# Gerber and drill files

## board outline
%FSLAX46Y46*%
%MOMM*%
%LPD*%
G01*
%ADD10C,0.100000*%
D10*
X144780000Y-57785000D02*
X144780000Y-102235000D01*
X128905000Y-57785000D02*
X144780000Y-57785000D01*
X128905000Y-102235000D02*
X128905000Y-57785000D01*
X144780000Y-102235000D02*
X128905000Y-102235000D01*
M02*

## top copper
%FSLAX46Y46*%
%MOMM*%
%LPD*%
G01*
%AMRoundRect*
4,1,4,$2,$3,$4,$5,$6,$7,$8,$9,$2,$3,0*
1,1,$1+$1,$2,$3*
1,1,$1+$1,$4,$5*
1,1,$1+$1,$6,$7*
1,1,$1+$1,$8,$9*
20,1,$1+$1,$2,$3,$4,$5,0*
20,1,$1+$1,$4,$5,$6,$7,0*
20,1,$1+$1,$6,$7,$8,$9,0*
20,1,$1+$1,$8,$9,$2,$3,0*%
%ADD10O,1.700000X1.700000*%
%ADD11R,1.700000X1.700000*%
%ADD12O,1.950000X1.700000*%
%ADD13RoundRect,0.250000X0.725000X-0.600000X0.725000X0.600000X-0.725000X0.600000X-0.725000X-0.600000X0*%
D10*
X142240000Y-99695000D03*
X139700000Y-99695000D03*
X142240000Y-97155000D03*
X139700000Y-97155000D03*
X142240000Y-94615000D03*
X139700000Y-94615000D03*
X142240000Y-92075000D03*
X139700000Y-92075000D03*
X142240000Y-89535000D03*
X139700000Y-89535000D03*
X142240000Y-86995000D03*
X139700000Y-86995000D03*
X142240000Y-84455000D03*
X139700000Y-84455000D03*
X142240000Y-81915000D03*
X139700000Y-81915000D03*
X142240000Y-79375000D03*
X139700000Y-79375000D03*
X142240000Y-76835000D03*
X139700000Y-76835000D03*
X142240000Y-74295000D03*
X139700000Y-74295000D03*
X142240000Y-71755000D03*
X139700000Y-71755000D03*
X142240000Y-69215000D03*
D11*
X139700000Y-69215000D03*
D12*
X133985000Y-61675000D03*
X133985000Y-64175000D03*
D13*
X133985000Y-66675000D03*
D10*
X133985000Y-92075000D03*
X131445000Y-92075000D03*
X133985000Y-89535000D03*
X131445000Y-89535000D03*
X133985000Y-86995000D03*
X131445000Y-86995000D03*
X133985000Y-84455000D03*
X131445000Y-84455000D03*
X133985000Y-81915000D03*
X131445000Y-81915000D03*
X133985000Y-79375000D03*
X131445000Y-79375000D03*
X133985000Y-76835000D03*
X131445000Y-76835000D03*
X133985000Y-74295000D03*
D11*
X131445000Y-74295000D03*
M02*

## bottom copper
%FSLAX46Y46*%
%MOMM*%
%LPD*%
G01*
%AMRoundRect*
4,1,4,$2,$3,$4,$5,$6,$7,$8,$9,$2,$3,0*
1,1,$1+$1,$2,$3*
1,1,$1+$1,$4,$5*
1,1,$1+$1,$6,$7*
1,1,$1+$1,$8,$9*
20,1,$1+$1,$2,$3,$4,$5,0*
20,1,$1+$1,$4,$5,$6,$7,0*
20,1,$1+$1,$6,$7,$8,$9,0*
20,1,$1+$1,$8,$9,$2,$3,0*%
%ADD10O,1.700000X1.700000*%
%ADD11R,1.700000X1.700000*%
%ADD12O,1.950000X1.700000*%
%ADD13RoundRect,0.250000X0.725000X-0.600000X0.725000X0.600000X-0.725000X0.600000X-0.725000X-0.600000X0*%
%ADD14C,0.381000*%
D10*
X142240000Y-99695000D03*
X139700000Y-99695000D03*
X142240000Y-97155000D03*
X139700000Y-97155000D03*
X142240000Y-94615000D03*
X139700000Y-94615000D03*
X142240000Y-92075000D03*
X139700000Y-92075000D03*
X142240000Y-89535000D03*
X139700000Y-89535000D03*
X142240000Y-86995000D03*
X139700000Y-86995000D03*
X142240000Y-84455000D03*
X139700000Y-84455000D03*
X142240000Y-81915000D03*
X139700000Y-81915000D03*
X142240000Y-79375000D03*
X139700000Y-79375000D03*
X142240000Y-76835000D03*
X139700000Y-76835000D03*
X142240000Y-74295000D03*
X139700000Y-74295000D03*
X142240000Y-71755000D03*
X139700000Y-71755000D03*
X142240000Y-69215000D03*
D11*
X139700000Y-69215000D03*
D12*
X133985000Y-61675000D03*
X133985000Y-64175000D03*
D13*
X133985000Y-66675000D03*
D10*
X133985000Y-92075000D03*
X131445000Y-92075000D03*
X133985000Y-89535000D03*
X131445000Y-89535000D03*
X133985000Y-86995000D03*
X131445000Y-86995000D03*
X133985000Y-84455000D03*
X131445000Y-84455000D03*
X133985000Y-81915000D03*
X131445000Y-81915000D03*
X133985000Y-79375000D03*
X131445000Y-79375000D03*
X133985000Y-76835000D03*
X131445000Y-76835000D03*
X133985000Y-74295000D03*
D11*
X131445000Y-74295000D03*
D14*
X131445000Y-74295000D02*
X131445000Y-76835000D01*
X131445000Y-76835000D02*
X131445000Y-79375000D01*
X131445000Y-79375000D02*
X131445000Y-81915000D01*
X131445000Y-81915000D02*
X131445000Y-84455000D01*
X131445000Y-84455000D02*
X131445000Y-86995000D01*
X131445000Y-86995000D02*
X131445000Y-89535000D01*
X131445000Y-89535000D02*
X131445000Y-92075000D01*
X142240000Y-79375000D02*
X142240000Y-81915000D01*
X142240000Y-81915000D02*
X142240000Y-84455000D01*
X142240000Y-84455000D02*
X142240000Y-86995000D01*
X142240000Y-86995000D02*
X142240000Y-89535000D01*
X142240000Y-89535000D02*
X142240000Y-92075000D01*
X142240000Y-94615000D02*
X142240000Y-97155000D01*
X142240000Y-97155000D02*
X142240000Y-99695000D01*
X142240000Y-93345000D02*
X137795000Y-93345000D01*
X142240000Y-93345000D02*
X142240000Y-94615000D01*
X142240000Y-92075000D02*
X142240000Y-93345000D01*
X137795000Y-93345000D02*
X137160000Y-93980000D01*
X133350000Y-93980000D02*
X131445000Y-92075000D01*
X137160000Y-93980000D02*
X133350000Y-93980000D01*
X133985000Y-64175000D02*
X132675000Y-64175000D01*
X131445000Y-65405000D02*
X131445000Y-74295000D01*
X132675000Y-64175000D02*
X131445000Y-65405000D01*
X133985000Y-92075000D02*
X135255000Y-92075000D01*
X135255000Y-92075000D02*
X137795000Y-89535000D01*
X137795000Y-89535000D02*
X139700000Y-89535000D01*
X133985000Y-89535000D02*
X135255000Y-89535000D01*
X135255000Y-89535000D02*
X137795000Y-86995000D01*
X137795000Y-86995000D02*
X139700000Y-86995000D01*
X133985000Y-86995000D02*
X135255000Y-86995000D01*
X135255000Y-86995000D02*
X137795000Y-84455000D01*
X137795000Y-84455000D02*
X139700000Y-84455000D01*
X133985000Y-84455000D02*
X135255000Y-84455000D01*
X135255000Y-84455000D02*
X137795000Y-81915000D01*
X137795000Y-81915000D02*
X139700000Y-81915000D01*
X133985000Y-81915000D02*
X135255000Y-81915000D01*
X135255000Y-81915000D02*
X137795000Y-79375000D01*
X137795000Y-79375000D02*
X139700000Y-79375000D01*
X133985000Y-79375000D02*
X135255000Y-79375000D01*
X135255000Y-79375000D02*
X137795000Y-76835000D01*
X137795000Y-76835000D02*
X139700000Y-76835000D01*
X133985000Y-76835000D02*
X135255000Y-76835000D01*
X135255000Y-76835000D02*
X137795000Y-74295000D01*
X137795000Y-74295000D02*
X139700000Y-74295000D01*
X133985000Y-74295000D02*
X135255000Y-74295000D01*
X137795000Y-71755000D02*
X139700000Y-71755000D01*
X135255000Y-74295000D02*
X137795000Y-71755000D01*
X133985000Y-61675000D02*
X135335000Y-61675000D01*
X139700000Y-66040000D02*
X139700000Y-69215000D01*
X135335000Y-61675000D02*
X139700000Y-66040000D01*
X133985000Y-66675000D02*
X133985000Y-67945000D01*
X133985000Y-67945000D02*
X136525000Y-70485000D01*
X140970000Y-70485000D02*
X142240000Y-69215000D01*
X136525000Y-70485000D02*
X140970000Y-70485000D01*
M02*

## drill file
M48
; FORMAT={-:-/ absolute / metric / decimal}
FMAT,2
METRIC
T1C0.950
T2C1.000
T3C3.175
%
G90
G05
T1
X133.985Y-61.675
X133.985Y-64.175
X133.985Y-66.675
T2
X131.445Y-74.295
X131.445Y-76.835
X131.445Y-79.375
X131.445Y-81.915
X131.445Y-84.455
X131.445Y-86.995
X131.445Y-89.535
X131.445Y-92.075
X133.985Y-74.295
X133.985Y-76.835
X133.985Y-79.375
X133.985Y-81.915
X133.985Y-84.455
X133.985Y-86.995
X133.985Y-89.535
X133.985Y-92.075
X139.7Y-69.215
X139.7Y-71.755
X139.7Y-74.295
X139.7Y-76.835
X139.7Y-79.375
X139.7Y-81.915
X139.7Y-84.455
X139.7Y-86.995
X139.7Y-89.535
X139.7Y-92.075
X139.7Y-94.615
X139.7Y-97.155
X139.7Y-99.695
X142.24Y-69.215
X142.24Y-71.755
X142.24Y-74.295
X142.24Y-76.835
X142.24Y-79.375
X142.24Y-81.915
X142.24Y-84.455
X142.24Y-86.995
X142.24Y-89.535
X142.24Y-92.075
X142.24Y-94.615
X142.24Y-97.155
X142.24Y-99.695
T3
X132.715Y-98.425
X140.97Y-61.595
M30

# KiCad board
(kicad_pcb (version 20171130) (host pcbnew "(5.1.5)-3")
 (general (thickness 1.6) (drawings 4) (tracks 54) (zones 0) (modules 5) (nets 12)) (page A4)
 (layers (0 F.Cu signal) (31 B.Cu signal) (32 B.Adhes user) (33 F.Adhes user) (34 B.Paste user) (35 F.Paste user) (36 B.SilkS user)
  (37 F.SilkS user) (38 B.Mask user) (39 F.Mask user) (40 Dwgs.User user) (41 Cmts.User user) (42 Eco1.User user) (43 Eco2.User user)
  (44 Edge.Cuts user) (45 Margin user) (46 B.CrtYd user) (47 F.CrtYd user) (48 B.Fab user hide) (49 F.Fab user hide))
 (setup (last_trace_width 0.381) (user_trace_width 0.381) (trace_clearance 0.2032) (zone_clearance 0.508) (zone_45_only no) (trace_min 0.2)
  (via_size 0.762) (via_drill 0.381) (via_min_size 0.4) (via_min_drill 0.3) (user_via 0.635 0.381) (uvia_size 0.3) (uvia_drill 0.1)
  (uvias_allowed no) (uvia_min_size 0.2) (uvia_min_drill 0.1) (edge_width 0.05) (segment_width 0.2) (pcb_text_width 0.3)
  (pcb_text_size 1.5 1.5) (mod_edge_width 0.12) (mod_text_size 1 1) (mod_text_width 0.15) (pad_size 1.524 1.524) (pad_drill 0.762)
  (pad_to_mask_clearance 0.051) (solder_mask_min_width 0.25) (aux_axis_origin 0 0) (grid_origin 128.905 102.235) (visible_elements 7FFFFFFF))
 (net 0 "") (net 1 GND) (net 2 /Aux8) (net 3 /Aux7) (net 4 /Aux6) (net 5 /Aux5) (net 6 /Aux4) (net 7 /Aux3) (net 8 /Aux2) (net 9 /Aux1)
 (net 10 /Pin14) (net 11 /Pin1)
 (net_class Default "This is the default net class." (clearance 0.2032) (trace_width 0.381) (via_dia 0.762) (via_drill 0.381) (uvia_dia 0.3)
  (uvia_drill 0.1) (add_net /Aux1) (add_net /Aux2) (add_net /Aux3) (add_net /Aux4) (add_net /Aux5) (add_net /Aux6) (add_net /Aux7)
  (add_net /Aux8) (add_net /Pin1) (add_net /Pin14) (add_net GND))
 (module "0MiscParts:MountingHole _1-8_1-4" (layer F.Cu) (at 132.715 98.425)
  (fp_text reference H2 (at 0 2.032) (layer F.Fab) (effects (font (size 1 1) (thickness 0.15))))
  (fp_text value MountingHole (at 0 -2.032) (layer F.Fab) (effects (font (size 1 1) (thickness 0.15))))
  (pad "" np_thru_hole circle (at 0 0) (size 3.175 3.175) (drill 3.175) (layers *.Cu *.Mask)))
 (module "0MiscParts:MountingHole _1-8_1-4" (layer F.Cu) (at 140.97 61.595)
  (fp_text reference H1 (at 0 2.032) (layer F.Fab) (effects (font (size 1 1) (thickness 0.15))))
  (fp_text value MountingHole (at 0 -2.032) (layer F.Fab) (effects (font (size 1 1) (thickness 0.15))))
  (pad "" np_thru_hole circle (at 0 0) (size 3.175 3.175) (drill 3.175) (layers *.Cu *.Mask)))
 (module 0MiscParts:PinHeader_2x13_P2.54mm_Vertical (layer F.Cu) (at 139.7 69.215)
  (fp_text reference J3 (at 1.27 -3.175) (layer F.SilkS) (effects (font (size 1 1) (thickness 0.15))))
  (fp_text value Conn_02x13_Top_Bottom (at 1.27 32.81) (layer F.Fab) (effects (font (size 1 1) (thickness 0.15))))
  (pad 26 thru_hole oval (at 2.54 30.48) (size 1.7 1.7) (drill 1) (layers *.Cu *.Mask) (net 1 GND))
  (pad 13 thru_hole oval (at 0 30.48) (size 1.7 1.7) (drill 1) (layers *.Cu *.Mask))
  (pad 25 thru_hole oval (at 2.54 27.94) (size 1.7 1.7) (drill 1) (layers *.Cu *.Mask) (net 1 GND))
  (pad 12 thru_hole oval (at 0 27.94) (size 1.7 1.7) (drill 1) (layers *.Cu *.Mask))
  (pad 24 thru_hole oval (at 2.54 25.4) (size 1.7 1.7) (drill 1) (layers *.Cu *.Mask) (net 1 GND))
  (pad 11 thru_hole oval (at 0 25.4) (size 1.7 1.7) (drill 1) (layers *.Cu *.Mask))
  (pad 23 thru_hole oval (at 2.54 22.86) (size 1.7 1.7) (drill 1) (layers *.Cu *.Mask) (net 1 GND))
  (pad 10 thru_hole oval (at 0 22.86) (size 1.7 1.7) (drill 1) (layers *.Cu *.Mask))
  (pad 22 thru_hole oval (at 2.54 20.32) (size 1.7 1.7) (drill 1) (layers *.Cu *.Mask) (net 1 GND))
  (pad 9 thru_hole oval (at 0 20.32) (size 1.7 1.7) (drill 1) (layers *.Cu *.Mask) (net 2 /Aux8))
  (pad 21 thru_hole oval (at 2.54 17.78) (size 1.7 1.7) (drill 1) (layers *.Cu *.Mask) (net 1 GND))
  (pad 8 thru_hole oval (at 0 17.78) (size 1.7 1.7) (drill 1) (layers *.Cu *.Mask) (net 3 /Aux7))
  (pad 20 thru_hole oval (at 2.54 15.24) (size 1.7 1.7) (drill 1) (layers *.Cu *.Mask) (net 1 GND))
  (pad 7 thru_hole oval (at 0 15.24) (size 1.7 1.7) (drill 1) (layers *.Cu *.Mask) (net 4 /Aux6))
  (pad 19 thru_hole oval (at 2.54 12.7) (size 1.7 1.7) (drill 1) (layers *.Cu *.Mask) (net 1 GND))
  (pad 6 thru_hole oval (at 0 12.7) (size 1.7 1.7) (drill 1) (layers *.Cu *.Mask) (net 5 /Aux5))
  (pad 18 thru_hole oval (at 2.54 10.16) (size 1.7 1.7) (drill 1) (layers *.Cu *.Mask) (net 1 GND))
  (pad 5 thru_hole oval (at 0 10.16) (size 1.7 1.7) (drill 1) (layers *.Cu *.Mask) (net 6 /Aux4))
  (pad 17 thru_hole oval (at 2.54 7.62) (size 1.7 1.7) (drill 1) (layers *.Cu *.Mask))
  (pad 4 thru_hole oval (at 0 7.62) (size 1.7 1.7) (drill 1) (layers *.Cu *.Mask) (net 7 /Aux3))
  (pad 16 thru_hole oval (at 2.54 5.08) (size 1.7 1.7) (drill 1) (layers *.Cu *.Mask))
  (pad 3 thru_hole oval (at 0 5.08) (size 1.7 1.7) (drill 1) (layers *.Cu *.Mask) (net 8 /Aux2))
  (pad 15 thru_hole oval (at 2.54 2.54) (size 1.7 1.7) (drill 1) (layers *.Cu *.Mask))
  (pad 2 thru_hole oval (at 0 2.54) (size 1.7 1.7) (drill 1) (layers *.Cu *.Mask) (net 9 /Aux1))
  (pad 14 thru_hole oval (at 2.54 0) (size 1.7 1.7) (drill 1) (layers *.Cu *.Mask) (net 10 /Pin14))
  (pad 1 thru_hole rect (at 0 0) (size 1.7 1.7) (drill 1) (layers *.Cu *.Mask) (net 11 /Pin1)))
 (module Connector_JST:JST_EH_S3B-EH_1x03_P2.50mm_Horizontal (layer F.Cu) (at 133.985 66.675 90)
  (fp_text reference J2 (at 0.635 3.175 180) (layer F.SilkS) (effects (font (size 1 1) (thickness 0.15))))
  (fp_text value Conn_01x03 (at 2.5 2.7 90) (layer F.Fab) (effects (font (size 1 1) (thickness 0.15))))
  (pad 3 thru_hole oval (at 5 0 90) (size 1.7 1.95) (drill 0.95) (layers *.Cu *.Mask) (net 11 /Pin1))
  (pad 2 thru_hole oval (at 2.5 0 90) (size 1.7 1.95) (drill 0.95) (layers *.Cu *.Mask) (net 1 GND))
  (pad 1 thru_hole roundrect (at 0 0 90) (size 1.7 1.95) (drill 0.95) (layers *.Cu *.Mask) (roundrect_rratio 0.147059) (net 10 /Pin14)))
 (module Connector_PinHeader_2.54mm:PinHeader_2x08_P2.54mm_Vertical (layer F.Cu) (at 131.445 74.295)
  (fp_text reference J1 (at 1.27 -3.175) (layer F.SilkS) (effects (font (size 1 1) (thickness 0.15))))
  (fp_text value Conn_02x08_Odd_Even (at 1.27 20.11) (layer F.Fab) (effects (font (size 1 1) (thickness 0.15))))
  (pad 16 thru_hole oval (at 2.54 17.78) (size 1.7 1.7) (drill 1) (layers *.Cu *.Mask) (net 2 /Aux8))
  (pad 15 thru_hole oval (at 0 17.78) (size 1.7 1.7) (drill 1) (layers *.Cu *.Mask) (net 1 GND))
  (pad 14 thru_hole oval (at 2.54 15.24) (size 1.7 1.7) (drill 1) (layers *.Cu *.Mask) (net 3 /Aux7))
  (pad 13 thru_hole oval (at 0 15.24) (size 1.7 1.7) (drill 1) (layers *.Cu *.Mask) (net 1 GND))
  (pad 12 thru_hole oval (at 2.54 12.7) (size 1.7 1.7) (drill 1) (layers *.Cu *.Mask) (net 4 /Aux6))
  (pad 11 thru_hole oval (at 0 12.7) (size 1.7 1.7) (drill 1) (layers *.Cu *.Mask) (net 1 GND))
  (pad 10 thru_hole oval (at 2.54 10.16) (size 1.7 1.7) (drill 1) (layers *.Cu *.Mask) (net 5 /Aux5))
  (pad 9 thru_hole oval (at 0 10.16) (size 1.7 1.7) (drill 1) (layers *.Cu *.Mask) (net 1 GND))
  (pad 8 thru_hole oval (at 2.54 7.62) (size 1.7 1.7) (drill 1) (layers *.Cu *.Mask) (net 6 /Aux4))
  (pad 7 thru_hole oval (at 0 7.62) (size 1.7 1.7) (drill 1) (layers *.Cu *.Mask) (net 1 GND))
  (pad 6 thru_hole oval (at 2.54 5.08) (size 1.7 1.7) (drill 1) (layers *.Cu *.Mask) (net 7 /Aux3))
  (pad 5 thru_hole oval (at 0 5.08) (size 1.7 1.7) (drill 1) (layers *.Cu *.Mask) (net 1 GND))
  (pad 4 thru_hole oval (at 2.54 2.54) (size 1.7 1.7) (drill 1) (layers *.Cu *.Mask) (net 8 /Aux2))
  (pad 3 thru_hole oval (at 0 2.54) (size 1.7 1.7) (drill 1) (layers *.Cu *.Mask) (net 1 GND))
  (pad 2 thru_hole oval (at 2.54 0) (size 1.7 1.7) (drill 1) (layers *.Cu *.Mask) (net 9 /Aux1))
  (pad 1 thru_hole rect (at 0 0) (size 1.7 1.7) (drill 1) (layers *.Cu *.Mask) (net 1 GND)))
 (gr_line (start 144.78 57.785) (end 144.78 102.235) (layer Edge.Cuts) (width 0.1))
 (gr_line (start 128.905 57.785) (end 144.78 57.785) (layer Edge.Cuts) (width 0.1))
 (gr_line (start 128.905 102.235) (end 128.905 57.785) (layer Edge.Cuts) (width 0.1))
 (gr_line (start 144.78 102.235) (end 128.905 102.235) (layer Edge.Cuts) (width 0.1))
 (segment (start 131.445 74.295) (end 131.445 76.835) (width 0.381) (layer B.Cu) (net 1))
 (segment (start 131.445 76.835) (end 131.445 79.375) (width 0.381) (layer B.Cu) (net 1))
 (segment (start 131.445 79.375) (end 131.445 81.915) (width 0.381) (layer B.Cu) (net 1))
 (segment (start 131.445 81.915) (end 131.445 84.455) (width 0.381) (layer B.Cu) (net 1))
 (segment (start 131.445 84.455) (end 131.445 86.995) (width 0.381) (layer B.Cu) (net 1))
 (segment (start 131.445 86.995) (end 131.445 89.535) (width 0.381) (layer B.Cu) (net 1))
 (segment (start 131.445 89.535) (end 131.445 92.075) (width 0.381) (layer B.Cu) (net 1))
 (segment (start 142.24 79.375) (end 142.24 81.915) (width 0.381) (layer B.Cu) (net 1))
 (segment (start 142.24 81.915) (end 142.24 84.455) (width 0.381) (layer B.Cu) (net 1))
 (segment (start 142.24 84.455) (end 142.24 86.995) (width 0.381) (layer B.Cu) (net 1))
 (segment (start 142.24 86.995) (end 142.24 89.535) (width 0.381) (layer B.Cu) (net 1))
 (segment (start 142.24 89.535) (end 142.24 92.075) (width 0.381) (layer B.Cu) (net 1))
 (segment (start 142.24 94.615) (end 142.24 97.155) (width 0.381) (layer B.Cu) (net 1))
 (segment (start 142.24 97.155) (end 142.24 99.695) (width 0.381) (layer B.Cu) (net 1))
 (segment (start 142.24 93.345) (end 137.795 93.345) (width 0.381) (layer B.Cu) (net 1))
 (segment (start 142.24 93.345) (end 142.24 94.615) (width 0.381) (layer B.Cu) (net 1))
 (segment (start 142.24 92.075) (end 142.24 93.345) (width 0.381) (layer B.Cu) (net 1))
 (segment (start 137.795 93.345) (end 137.16 93.98) (width 0.381) (layer B.Cu) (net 1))
 (segment (start 133.35 93.98) (end 131.445 92.075) (width 0.381) (layer B.Cu) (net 1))
 (segment (start 137.16 93.98) (end 133.35 93.98) (width 0.381) (layer B.Cu) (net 1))
 (segment (start 133.985 64.175) (end 132.675 64.175) (width 0.381) (layer B.Cu) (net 1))
 (segment (start 131.445 65.405) (end 131.445 74.295) (width 0.381) (layer B.Cu) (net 1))
 (segment (start 132.675 64.175) (end 131.445 65.405) (width 0.381) (layer B.Cu) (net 1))
 (segment (start 133.985 92.075) (end 135.255 92.075) (width 0.381) (layer B.Cu) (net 2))
 (segment (start 135.255 92.075) (end 137.795 89.535) (width 0.381) (layer B.Cu) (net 2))
 (segment (start 137.795 89.535) (end 139.7 89.535) (width 0.381) (layer B.Cu) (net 2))
 (segment (start 133.985 89.535) (end 135.255 89.535) (width 0.381) (layer B.Cu) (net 3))
 (segment (start 135.255 89.535) (end 137.795 86.995) (width 0.381) (layer B.Cu) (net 3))
 (segment (start 137.795 86.995) (end 139.7 86.995) (width 0.381) (layer B.Cu) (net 3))
 (segment (start 133.985 86.995) (end 135.255 86.995) (width 0.381) (layer B.Cu) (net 4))
 (segment (start 135.255 86.995) (end 137.795 84.455) (width 0.381) (layer B.Cu) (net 4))
 (segment (start 137.795 84.455) (end 139.7 84.455) (width 0.381) (layer B.Cu) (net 4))
 (segment (start 133.985 84.455) (end 135.255 84.455) (width 0.381) (layer B.Cu) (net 5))
 (segment (start 135.255 84.455) (end 137.795 81.915) (width 0.381) (layer B.Cu) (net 5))
 (segment (start 137.795 81.915) (end 139.7 81.915) (width 0.381) (layer B.Cu) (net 5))
 (segment (start 133.985 81.915) (end 135.255 81.915) (width 0.381) (layer B.Cu) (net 6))
 (segment (start 135.255 81.915) (end 137.795 79.375) (width 0.381) (layer B.Cu) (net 6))
 (segment (start 137.795 79.375) (end 139.7 79.375) (width 0.381) (layer B.Cu) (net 6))
 (segment (start 133.985 79.375) (end 135.255 79.375) (width 0.381) (layer B.Cu) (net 7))
 (segment (start 135.255 79.375) (end 137.795 76.835) (width 0.381) (layer B.Cu) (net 7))
 (segment (start 137.795 76.835) (end 139.7 76.835) (width 0.381) (layer B.Cu) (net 7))
 (segment (start 133.985 76.835) (end 135.255 76.835) (width 0.381) (layer B.Cu) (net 8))
 (segment (start 135.255 76.835) (end 137.795 74.295) (width 0.381) (layer B.Cu) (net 8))
 (segment (start 137.795 74.295) (end 139.7 74.295) (width 0.381) (layer B.Cu) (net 8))
 (segment (start 133.985 74.295) (end 135.255 74.295) (width 0.381) (layer B.Cu) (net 9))
 (segment (start 137.795 71.755) (end 139.7 71.755) (width 0.381) (layer B.Cu) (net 9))
 (segment (start 135.255 74.295) (end 137.795 71.755) (width 0.381) (layer B.Cu) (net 9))
 (segment (start 133.985 61.675) (end 135.335 61.675) (width 0.381) (layer B.Cu) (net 11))
 (segment (start 139.7 66.04) (end 139.7 69.215) (width 0.381) (layer B.Cu) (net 11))
 (segment (start 135.335 61.675) (end 139.7 66.04) (width 0.381) (layer B.Cu) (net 11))
 (segment (start 133.985 66.675) (end 133.985 67.945) (width 0.381) (layer B.Cu) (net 10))
 (segment (start 133.985 67.945) (end 136.525 70.485) (width 0.381) (layer B.Cu) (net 10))
 (segment (start 140.97 70.485) (end 142.24 69.215) (width 0.381) (layer B.Cu) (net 10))
 (segment (start 136.525 70.485) (end 140.97 70.485) (width 0.381) (layer B.Cu) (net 10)))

